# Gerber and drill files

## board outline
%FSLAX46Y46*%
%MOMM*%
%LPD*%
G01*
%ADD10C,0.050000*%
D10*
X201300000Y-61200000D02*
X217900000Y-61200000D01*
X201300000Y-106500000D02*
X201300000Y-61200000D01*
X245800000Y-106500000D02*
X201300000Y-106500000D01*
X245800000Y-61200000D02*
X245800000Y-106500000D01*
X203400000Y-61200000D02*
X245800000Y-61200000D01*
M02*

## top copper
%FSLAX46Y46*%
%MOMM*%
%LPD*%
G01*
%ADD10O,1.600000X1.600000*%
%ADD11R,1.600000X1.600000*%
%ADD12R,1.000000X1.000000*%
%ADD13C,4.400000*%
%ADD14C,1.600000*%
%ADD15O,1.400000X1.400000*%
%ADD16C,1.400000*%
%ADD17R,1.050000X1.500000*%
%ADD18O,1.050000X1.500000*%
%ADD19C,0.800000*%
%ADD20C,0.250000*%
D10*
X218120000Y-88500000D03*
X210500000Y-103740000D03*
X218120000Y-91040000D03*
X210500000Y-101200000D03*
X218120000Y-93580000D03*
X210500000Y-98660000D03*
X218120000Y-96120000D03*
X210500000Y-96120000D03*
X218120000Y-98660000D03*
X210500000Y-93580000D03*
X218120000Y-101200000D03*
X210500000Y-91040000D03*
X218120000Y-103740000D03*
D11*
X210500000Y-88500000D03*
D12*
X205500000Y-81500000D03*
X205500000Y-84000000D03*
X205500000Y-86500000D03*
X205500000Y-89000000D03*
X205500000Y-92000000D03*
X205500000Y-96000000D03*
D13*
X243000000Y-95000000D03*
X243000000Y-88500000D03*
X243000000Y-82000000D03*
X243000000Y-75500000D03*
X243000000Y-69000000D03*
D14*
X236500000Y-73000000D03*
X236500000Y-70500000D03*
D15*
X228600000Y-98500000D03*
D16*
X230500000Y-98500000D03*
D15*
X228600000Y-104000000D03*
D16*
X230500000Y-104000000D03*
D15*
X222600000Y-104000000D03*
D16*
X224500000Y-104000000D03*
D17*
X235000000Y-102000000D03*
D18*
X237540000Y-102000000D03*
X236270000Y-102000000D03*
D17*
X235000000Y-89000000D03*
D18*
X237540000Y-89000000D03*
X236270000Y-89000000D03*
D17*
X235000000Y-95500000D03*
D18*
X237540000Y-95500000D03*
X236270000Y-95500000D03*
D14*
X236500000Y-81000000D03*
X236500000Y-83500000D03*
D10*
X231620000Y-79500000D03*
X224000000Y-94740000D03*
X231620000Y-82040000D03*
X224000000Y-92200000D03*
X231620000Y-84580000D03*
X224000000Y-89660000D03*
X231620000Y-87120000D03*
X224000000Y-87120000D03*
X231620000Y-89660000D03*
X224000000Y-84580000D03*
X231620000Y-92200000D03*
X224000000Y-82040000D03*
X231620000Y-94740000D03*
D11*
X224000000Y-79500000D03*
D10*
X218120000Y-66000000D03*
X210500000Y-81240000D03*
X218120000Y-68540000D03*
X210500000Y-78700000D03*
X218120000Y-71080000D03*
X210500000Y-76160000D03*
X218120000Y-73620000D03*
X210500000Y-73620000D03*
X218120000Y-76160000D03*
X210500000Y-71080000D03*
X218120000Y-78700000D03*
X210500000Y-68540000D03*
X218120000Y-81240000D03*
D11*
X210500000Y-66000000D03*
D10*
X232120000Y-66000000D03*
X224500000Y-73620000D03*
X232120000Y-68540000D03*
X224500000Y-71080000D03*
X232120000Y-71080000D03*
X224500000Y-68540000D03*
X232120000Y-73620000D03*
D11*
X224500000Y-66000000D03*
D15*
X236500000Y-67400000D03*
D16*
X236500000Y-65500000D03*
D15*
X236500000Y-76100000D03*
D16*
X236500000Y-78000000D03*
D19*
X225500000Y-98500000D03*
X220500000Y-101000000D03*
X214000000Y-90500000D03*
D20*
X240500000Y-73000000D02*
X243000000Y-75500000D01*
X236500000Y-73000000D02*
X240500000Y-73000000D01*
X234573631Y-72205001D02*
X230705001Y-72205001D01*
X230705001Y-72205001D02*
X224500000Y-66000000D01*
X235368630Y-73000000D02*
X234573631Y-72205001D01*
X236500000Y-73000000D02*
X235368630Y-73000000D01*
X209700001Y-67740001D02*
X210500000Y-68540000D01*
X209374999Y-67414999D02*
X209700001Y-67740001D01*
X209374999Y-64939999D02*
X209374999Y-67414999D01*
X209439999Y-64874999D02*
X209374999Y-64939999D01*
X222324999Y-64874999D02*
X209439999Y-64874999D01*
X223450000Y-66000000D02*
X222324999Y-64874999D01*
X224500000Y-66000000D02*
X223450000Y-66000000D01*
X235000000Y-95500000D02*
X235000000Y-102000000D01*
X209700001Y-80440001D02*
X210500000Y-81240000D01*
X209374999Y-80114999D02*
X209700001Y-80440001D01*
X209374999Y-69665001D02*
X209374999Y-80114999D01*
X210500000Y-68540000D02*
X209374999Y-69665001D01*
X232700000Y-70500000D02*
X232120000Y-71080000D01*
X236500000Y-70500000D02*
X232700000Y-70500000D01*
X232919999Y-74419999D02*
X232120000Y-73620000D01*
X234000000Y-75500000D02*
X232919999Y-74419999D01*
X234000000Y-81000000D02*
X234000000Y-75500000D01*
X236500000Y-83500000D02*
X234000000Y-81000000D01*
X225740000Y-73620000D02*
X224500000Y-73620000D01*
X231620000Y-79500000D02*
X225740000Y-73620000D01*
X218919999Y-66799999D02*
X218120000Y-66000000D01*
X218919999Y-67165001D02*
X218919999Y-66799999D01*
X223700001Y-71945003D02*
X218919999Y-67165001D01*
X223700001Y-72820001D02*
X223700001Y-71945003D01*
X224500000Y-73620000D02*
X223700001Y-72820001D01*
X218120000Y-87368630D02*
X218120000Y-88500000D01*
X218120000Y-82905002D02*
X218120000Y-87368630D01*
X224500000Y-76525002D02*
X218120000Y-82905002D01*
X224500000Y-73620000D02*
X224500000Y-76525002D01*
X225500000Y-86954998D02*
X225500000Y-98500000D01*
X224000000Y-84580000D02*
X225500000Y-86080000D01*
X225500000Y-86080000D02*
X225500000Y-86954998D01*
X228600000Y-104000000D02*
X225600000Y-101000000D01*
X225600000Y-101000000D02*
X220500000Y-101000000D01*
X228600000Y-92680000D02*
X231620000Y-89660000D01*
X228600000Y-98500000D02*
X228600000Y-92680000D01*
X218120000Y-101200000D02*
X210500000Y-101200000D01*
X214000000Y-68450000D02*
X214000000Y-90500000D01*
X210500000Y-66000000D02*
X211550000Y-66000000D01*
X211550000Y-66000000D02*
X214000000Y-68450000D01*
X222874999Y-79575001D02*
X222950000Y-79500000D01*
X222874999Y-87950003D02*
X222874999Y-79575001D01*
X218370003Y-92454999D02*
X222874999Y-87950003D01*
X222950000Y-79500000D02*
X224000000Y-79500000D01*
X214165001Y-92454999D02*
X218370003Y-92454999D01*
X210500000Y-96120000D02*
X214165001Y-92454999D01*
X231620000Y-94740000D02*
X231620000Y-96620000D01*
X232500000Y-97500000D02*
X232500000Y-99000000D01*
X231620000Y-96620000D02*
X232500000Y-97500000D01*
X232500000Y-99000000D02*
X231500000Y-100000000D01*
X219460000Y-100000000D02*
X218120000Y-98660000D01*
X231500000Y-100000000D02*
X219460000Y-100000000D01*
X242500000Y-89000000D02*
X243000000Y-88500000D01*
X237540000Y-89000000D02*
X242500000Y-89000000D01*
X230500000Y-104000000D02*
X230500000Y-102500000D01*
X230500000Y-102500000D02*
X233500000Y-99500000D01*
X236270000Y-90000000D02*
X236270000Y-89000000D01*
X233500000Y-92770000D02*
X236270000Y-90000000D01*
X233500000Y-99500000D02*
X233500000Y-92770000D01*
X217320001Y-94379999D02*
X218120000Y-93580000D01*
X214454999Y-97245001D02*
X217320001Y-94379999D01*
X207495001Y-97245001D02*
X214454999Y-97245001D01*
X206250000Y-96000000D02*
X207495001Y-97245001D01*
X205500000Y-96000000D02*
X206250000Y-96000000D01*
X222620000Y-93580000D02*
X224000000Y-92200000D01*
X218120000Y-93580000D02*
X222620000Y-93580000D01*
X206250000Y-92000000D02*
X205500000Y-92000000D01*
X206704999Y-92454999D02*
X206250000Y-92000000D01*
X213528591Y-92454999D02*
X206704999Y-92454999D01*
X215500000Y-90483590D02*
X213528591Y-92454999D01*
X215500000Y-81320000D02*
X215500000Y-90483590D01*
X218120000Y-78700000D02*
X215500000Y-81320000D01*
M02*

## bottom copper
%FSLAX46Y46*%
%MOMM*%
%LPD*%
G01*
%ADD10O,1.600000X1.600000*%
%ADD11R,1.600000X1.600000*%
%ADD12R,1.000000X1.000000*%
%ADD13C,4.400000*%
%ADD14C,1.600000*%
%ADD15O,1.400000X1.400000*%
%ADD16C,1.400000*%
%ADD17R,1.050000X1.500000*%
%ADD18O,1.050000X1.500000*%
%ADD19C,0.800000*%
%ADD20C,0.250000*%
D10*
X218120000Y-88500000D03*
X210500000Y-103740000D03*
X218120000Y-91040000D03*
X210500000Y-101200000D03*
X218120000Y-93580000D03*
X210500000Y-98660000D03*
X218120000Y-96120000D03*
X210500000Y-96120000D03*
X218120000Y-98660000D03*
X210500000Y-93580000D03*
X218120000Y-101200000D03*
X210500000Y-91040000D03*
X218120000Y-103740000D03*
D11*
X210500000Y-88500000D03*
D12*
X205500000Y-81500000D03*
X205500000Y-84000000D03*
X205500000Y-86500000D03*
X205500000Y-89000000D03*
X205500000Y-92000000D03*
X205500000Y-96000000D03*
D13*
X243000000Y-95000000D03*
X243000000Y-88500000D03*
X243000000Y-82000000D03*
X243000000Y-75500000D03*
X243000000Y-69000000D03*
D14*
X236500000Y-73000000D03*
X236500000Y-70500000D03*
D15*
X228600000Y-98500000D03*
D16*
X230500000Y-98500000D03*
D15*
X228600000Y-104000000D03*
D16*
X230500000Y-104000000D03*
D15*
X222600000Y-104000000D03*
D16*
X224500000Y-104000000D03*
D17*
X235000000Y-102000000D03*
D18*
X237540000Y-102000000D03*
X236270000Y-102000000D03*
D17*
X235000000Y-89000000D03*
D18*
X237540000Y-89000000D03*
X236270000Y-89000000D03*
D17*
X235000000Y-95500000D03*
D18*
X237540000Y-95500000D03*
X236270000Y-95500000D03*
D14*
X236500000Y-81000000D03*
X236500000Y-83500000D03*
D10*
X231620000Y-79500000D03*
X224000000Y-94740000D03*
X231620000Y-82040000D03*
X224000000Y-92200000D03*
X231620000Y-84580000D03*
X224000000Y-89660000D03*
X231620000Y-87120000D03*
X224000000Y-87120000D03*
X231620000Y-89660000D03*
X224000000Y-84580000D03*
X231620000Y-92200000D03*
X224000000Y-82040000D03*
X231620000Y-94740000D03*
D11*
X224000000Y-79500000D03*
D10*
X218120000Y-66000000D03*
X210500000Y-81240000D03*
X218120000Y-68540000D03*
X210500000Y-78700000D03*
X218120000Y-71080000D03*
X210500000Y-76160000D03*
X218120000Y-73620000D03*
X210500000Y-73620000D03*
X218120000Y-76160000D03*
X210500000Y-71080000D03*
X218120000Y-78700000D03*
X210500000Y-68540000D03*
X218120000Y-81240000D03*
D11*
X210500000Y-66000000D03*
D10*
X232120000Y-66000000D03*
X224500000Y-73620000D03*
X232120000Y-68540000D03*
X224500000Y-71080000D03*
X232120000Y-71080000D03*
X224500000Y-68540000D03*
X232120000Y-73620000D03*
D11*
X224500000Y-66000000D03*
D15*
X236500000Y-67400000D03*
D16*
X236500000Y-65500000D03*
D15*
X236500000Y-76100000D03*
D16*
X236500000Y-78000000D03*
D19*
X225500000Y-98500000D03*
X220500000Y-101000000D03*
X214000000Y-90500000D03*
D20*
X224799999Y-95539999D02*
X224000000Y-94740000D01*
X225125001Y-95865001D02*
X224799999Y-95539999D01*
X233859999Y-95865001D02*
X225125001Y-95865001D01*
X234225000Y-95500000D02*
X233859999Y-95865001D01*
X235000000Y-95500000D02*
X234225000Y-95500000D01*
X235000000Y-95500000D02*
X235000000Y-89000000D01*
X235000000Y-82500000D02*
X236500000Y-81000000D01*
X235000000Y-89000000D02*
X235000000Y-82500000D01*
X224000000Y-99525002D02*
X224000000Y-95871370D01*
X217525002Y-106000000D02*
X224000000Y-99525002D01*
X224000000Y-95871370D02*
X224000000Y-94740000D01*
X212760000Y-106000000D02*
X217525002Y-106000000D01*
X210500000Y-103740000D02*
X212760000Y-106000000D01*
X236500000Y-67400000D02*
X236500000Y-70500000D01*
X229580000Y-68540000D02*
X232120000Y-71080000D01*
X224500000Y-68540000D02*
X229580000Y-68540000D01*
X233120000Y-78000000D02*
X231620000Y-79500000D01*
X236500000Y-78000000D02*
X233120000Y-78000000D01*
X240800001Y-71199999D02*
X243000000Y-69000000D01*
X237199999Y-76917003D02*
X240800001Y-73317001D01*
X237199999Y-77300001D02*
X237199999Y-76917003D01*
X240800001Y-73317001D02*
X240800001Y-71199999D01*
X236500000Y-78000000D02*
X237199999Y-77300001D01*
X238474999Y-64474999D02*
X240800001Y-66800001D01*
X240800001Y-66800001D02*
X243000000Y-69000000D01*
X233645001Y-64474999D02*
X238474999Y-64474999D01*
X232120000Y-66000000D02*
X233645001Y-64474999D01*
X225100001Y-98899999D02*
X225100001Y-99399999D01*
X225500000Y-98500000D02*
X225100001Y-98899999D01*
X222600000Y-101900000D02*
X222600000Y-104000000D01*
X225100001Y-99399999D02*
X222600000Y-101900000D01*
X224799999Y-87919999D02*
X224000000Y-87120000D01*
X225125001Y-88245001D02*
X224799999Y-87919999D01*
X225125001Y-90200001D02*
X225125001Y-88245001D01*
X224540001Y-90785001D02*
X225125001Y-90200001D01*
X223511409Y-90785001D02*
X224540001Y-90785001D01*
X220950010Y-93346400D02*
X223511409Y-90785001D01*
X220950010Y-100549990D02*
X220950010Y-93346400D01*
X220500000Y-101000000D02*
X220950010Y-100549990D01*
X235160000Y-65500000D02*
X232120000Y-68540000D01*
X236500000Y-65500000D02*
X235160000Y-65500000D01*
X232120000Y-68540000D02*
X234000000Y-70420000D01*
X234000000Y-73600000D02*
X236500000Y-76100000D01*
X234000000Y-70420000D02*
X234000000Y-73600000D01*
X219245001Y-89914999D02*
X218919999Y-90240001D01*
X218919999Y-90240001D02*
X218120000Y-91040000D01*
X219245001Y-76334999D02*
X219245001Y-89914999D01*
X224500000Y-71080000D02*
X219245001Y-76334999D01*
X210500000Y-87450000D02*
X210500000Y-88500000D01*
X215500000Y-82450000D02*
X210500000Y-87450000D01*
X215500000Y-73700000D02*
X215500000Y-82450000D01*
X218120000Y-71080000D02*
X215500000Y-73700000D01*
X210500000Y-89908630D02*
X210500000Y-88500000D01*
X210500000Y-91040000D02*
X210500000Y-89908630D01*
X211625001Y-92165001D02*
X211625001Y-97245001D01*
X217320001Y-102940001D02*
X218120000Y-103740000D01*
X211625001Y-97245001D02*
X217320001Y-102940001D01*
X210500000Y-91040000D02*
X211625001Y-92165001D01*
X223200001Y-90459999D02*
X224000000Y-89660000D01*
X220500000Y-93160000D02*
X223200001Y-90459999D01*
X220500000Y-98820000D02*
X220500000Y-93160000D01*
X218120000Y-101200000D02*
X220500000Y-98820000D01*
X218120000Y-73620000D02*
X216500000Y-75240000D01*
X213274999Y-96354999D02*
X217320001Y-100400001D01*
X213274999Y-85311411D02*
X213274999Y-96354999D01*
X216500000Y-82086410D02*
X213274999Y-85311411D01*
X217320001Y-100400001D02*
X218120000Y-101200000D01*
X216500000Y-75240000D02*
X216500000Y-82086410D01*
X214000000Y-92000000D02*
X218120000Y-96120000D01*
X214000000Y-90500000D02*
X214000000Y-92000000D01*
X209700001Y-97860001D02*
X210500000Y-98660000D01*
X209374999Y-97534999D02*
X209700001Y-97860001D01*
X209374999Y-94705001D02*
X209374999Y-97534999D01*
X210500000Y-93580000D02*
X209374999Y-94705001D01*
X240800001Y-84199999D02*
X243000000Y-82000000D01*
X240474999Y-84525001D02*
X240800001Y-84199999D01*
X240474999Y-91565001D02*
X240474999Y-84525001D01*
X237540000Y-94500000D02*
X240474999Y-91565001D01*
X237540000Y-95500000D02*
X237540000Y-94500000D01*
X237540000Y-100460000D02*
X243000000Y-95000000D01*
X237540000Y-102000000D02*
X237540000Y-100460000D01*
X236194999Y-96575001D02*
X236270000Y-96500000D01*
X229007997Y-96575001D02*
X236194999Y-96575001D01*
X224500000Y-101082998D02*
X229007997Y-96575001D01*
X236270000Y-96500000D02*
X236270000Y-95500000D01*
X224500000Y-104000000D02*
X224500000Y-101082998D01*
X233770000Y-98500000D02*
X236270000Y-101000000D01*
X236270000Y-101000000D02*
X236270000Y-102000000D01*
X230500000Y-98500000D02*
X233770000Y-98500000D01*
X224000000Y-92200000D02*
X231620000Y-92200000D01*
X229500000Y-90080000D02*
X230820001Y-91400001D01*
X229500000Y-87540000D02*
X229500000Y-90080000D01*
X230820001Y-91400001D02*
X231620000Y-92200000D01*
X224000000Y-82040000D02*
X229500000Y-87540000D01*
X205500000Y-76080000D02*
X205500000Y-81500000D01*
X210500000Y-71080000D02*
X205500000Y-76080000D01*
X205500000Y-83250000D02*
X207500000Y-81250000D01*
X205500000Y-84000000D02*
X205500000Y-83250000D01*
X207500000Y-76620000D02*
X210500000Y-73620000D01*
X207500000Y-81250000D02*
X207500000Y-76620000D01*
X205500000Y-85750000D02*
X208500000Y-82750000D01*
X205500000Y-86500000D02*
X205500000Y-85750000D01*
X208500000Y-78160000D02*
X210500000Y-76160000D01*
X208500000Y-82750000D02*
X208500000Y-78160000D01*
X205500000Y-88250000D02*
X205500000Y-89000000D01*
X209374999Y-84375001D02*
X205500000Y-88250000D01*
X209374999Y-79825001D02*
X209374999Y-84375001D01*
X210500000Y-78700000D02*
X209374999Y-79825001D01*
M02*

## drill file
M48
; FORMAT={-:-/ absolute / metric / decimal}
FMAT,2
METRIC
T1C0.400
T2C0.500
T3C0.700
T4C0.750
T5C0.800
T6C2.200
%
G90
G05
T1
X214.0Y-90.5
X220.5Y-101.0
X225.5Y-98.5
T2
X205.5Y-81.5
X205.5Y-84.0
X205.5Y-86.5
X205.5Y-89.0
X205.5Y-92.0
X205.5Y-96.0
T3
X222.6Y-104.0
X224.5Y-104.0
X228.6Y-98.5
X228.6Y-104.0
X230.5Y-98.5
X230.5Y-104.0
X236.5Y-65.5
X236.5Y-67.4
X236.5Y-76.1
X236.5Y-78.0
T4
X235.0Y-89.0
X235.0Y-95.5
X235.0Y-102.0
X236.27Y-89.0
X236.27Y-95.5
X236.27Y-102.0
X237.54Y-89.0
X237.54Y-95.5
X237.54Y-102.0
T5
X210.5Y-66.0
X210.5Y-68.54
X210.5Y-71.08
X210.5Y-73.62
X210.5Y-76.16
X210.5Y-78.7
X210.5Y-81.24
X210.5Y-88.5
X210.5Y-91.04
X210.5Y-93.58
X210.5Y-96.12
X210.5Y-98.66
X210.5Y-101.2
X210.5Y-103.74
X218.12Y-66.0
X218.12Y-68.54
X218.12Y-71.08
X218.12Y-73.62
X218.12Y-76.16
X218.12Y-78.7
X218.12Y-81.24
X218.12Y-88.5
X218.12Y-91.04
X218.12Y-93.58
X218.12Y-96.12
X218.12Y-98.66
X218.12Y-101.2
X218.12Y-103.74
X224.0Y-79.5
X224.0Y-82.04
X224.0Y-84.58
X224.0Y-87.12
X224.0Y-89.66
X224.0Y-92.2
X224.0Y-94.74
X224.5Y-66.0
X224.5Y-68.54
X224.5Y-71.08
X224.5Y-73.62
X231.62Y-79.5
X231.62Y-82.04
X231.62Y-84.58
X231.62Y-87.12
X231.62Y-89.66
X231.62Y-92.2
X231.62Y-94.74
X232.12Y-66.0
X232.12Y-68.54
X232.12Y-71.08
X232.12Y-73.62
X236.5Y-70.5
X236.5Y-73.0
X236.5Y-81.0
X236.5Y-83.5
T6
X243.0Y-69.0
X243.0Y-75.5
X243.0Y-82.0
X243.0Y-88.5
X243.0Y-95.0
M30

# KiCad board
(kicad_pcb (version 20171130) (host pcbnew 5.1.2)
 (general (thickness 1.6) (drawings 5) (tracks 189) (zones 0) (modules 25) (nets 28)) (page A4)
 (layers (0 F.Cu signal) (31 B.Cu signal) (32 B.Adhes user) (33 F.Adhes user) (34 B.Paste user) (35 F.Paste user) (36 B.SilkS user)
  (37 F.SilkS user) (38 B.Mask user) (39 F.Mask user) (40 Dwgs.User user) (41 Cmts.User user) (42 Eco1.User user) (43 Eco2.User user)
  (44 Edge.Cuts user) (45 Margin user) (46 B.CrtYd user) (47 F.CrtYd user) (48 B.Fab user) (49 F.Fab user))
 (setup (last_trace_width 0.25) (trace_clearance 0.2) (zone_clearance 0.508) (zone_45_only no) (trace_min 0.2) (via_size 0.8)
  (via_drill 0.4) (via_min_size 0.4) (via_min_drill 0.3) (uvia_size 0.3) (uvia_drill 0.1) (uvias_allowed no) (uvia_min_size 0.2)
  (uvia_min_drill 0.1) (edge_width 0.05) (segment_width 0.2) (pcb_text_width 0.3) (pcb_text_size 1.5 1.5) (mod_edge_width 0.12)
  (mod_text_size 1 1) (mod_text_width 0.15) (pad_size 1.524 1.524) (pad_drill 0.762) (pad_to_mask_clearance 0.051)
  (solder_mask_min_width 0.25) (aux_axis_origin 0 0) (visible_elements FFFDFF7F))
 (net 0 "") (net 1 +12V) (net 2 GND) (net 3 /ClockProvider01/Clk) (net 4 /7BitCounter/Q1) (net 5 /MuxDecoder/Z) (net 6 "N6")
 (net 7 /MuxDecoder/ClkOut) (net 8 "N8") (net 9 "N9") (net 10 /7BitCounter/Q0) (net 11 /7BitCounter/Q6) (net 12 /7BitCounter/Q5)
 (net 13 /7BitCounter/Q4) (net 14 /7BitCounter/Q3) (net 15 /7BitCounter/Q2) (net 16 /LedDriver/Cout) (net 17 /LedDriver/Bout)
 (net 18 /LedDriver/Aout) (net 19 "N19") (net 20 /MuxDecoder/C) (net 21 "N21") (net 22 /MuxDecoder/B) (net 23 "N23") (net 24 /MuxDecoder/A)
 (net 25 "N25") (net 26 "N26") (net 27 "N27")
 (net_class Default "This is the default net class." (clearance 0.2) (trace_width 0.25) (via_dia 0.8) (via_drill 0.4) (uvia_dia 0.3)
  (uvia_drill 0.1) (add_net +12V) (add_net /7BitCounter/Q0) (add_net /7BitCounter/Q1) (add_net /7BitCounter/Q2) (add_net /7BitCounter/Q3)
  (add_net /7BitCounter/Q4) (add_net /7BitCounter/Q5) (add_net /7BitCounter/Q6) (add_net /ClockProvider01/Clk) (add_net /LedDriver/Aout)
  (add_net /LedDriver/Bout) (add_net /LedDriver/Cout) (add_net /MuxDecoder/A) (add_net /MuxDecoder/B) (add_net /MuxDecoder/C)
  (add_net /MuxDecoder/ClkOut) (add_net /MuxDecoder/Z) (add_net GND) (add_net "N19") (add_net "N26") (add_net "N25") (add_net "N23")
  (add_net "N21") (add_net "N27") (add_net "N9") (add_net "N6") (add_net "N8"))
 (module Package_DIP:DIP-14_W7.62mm (layer F.Cu) (at 210.5 88.5)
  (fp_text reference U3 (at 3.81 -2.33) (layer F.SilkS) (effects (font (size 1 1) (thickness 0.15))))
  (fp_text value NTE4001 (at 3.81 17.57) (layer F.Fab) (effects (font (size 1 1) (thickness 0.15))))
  (pad 14 thru_hole oval (at 7.62 0) (size 1.6 1.6) (drill 0.8) (layers *.Cu *.Mask) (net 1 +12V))
  (pad 7 thru_hole oval (at 0 15.24) (size 1.6 1.6) (drill 0.8) (layers *.Cu *.Mask) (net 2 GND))
  (pad 13 thru_hole oval (at 7.62 2.54) (size 1.6 1.6) (drill 0.8) (layers *.Cu *.Mask) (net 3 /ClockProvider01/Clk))
  (pad 6 thru_hole oval (at 0 12.7) (size 1.6 1.6) (drill 0.8) (layers *.Cu *.Mask) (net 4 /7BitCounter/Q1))
  (pad 12 thru_hole oval (at 7.62 5.08) (size 1.6 1.6) (drill 0.8) (layers *.Cu *.Mask) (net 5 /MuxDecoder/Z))
  (pad 5 thru_hole oval (at 0 10.16) (size 1.6 1.6) (drill 0.8) (layers *.Cu *.Mask) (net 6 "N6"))
  (pad 11 thru_hole oval (at 7.62 7.62) (size 1.6 1.6) (drill 0.8) (layers *.Cu *.Mask) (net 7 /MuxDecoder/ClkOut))
  (pad 4 thru_hole oval (at 0 7.62) (size 1.6 1.6) (drill 0.8) (layers *.Cu *.Mask) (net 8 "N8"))
  (pad 10 thru_hole oval (at 7.62 10.16) (size 1.6 1.6) (drill 0.8) (layers *.Cu *.Mask) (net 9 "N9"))
  (pad 3 thru_hole oval (at 0 5.08) (size 1.6 1.6) (drill 0.8) (layers *.Cu *.Mask) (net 6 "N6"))
  (pad 9 thru_hole oval (at 7.62 12.7) (size 1.6 1.6) (drill 0.8) (layers *.Cu *.Mask) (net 4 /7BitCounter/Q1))
  (pad 2 thru_hole oval (at 0 2.54) (size 1.6 1.6) (drill 0.8) (layers *.Cu *.Mask) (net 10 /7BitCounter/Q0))
  (pad 8 thru_hole oval (at 7.62 15.24) (size 1.6 1.6) (drill 0.8) (layers *.Cu *.Mask) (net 10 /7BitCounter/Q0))
  (pad 1 thru_hole rect (at 0 0) (size 1.6 1.6) (drill 0.8) (layers *.Cu *.Mask) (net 10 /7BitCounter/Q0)))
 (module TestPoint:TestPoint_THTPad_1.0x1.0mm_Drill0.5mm (layer F.Cu) (at 205.5 81.5 180)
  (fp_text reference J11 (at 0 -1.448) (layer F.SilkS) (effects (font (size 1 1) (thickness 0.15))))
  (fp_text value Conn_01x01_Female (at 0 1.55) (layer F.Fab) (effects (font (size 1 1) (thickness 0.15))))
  (pad 1 thru_hole rect (at 0 0 180) (size 1 1) (drill 0.5) (layers *.Cu *.Mask) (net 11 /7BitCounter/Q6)))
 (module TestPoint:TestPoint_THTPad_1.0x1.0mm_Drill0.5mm (layer F.Cu) (at 205.5 84 180)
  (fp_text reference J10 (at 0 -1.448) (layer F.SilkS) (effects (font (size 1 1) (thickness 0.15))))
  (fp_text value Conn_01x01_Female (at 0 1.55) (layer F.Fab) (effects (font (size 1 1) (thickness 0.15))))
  (pad 1 thru_hole rect (at 0 0 180) (size 1 1) (drill 0.5) (layers *.Cu *.Mask) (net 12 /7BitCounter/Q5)))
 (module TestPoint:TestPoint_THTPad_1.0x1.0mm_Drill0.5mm (layer F.Cu) (at 205.5 86.5 180)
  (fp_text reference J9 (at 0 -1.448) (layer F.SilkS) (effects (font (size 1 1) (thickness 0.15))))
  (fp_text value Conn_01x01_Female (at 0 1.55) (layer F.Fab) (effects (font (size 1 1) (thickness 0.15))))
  (pad 1 thru_hole rect (at 0 0 180) (size 1 1) (drill 0.5) (layers *.Cu *.Mask) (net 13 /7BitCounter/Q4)))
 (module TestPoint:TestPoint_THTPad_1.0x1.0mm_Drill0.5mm (layer F.Cu) (at 205.5 89 180)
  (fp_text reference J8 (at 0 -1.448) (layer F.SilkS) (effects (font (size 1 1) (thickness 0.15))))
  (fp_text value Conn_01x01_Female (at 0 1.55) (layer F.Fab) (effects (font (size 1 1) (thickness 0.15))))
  (pad 1 thru_hole rect (at 0 0 180) (size 1 1) (drill 0.5) (layers *.Cu *.Mask) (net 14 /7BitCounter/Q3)))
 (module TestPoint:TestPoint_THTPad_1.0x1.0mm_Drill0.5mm (layer F.Cu) (at 205.5 92 180)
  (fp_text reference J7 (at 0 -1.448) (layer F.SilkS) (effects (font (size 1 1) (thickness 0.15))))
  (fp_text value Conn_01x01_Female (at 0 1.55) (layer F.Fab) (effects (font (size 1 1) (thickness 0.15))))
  (pad 1 thru_hole rect (at 0 0 180) (size 1 1) (drill 0.5) (layers *.Cu *.Mask) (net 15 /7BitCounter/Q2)))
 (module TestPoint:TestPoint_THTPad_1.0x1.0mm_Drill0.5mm (layer F.Cu) (at 205.5 96 180)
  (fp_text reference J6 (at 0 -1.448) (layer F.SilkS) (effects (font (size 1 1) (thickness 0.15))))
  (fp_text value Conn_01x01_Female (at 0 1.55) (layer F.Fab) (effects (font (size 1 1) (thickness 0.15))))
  (pad 1 thru_hole rect (at 0 0 180) (size 1 1) (drill 0.5) (layers *.Cu *.Mask) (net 5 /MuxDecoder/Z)))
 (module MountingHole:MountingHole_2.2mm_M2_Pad (layer F.Cu) (at 243 95)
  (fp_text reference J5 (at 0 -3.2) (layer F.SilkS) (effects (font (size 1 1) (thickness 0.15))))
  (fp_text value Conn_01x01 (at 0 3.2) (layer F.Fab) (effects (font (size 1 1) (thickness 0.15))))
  (pad 1 thru_hole circle (at 0 0) (size 4.4 4.4) (drill 2.2) (layers *.Cu *.Mask) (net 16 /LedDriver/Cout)))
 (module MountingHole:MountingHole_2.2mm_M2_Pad (layer F.Cu) (at 243 88.5)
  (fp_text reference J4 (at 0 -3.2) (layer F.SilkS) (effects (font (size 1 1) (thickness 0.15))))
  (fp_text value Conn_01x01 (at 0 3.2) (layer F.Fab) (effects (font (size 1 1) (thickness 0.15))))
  (pad 1 thru_hole circle (at 0 0) (size 4.4 4.4) (drill 2.2) (layers *.Cu *.Mask) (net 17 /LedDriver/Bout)))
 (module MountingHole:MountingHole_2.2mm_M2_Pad (layer F.Cu) (at 243 82)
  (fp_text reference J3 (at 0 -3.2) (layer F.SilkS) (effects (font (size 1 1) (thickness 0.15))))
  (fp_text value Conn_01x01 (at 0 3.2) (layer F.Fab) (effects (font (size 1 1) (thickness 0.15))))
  (pad 1 thru_hole circle (at 0 0) (size 4.4 4.4) (drill 2.2) (layers *.Cu *.Mask) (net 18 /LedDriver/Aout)))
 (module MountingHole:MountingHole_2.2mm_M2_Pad (layer F.Cu) (at 243 75.5)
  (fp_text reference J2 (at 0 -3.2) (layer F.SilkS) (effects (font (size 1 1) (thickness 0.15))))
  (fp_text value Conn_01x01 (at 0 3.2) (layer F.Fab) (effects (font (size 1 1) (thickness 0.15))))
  (pad 1 thru_hole circle (at 0 0) (size 4.4 4.4) (drill 2.2) (layers *.Cu *.Mask) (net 2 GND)))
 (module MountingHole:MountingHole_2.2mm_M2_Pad (layer F.Cu) (at 243 69)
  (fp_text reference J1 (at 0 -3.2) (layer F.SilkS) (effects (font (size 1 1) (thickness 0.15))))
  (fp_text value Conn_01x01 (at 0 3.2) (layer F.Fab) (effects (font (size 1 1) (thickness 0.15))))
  (pad 1 thru_hole circle (at 0 0) (size 4.4 4.4) (drill 2.2) (layers *.Cu *.Mask) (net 1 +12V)))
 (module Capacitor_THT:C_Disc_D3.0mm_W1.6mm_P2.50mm (layer F.Cu) (at 236.5 70.5 270)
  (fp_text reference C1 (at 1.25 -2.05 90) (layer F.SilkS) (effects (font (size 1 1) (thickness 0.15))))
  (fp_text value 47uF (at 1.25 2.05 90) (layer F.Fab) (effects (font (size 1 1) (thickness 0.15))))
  (pad 2 thru_hole circle (at 2.5 0 270) (size 1.6 1.6) (drill 0.8) (layers *.Cu *.Mask) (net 2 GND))
  (pad 1 thru_hole circle (at 0 0 270) (size 1.6 1.6) (drill 0.8) (layers *.Cu *.Mask) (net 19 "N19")))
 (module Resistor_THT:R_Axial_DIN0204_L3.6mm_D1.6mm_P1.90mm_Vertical (layer F.Cu) (at 230.5 98.5 180)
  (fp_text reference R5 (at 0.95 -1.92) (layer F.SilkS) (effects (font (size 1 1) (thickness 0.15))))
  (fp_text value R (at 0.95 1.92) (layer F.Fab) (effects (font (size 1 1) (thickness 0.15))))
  (pad 2 thru_hole oval (at 1.9 0 180) (size 1.4 1.4) (drill 0.7) (layers *.Cu *.Mask) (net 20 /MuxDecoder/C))
  (pad 1 thru_hole circle (at 0 0 180) (size 1.4 1.4) (drill 0.7) (layers *.Cu *.Mask) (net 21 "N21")))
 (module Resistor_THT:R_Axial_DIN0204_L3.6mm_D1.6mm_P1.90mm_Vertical (layer F.Cu) (at 230.5 104 180)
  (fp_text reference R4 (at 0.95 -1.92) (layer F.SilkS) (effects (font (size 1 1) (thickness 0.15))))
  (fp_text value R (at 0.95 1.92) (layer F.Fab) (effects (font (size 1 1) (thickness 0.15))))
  (pad 2 thru_hole oval (at 1.9 0 180) (size 1.4 1.4) (drill 0.7) (layers *.Cu *.Mask) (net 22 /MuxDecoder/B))
  (pad 1 thru_hole circle (at 0 0 180) (size 1.4 1.4) (drill 0.7) (layers *.Cu *.Mask) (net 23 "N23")))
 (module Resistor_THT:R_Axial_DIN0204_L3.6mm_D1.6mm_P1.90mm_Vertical (layer F.Cu) (at 224.5 104 180)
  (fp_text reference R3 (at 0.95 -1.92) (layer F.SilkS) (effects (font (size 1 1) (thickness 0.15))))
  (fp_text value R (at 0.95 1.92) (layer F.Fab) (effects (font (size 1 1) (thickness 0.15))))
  (pad 2 thru_hole oval (at 1.9 0 180) (size 1.4 1.4) (drill 0.7) (layers *.Cu *.Mask) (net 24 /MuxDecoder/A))
  (pad 1 thru_hole circle (at 0 0 180) (size 1.4 1.4) (drill 0.7) (layers *.Cu *.Mask) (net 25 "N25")))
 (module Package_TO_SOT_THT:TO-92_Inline (layer F.Cu) (at 235 102)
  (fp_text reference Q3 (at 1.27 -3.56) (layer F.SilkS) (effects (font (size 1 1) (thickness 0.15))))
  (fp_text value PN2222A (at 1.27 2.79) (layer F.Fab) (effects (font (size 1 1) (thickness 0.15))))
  (pad 1 thru_hole rect (at 0 0) (size 1.05 1.5) (drill 0.75) (layers *.Cu *.Mask) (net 2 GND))
  (pad 3 thru_hole oval (at 2.54 0) (size 1.05 1.5) (drill 0.75) (layers *.Cu *.Mask) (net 16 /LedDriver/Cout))
  (pad 2 thru_hole oval (at 1.27 0) (size 1.05 1.5) (drill 0.75) (layers *.Cu *.Mask) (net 21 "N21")))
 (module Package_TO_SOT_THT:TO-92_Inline (layer F.Cu) (at 235 89)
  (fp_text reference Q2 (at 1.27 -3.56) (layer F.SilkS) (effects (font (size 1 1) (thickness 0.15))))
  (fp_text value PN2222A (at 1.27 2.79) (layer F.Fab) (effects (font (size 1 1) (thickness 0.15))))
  (pad 1 thru_hole rect (at 0 0) (size 1.05 1.5) (drill 0.75) (layers *.Cu *.Mask) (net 2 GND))
  (pad 3 thru_hole oval (at 2.54 0) (size 1.05 1.5) (drill 0.75) (layers *.Cu *.Mask) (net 17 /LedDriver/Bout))
  (pad 2 thru_hole oval (at 1.27 0) (size 1.05 1.5) (drill 0.75) (layers *.Cu *.Mask) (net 23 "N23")))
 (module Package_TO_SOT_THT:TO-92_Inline (layer F.Cu) (at 235 95.5)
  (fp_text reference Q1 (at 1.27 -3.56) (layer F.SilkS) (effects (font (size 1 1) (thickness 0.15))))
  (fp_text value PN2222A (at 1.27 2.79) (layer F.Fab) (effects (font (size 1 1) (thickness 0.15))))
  (pad 1 thru_hole rect (at 0 0) (size 1.05 1.5) (drill 0.75) (layers *.Cu *.Mask) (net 2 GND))
  (pad 3 thru_hole oval (at 2.54 0) (size 1.05 1.5) (drill 0.75) (layers *.Cu *.Mask) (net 18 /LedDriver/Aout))
  (pad 2 thru_hole oval (at 1.27 0) (size 1.05 1.5) (drill 0.75) (layers *.Cu *.Mask) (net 25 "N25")))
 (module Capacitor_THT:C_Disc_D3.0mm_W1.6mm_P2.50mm (layer F.Cu) (at 236.5 83.5 90)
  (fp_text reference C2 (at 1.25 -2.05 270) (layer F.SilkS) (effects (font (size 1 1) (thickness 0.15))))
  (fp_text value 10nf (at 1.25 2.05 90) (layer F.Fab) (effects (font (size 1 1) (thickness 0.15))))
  (pad 2 thru_hole circle (at 2.5 0 90) (size 1.6 1.6) (drill 0.8) (layers *.Cu *.Mask) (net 2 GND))
  (pad 1 thru_hole circle (at 0 0 90) (size 1.6 1.6) (drill 0.8) (layers *.Cu *.Mask) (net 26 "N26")))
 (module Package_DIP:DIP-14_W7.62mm (layer F.Cu) (at 224 79.5)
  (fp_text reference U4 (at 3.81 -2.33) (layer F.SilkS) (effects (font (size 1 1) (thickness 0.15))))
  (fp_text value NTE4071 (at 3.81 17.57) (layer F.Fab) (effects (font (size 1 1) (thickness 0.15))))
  (pad 14 thru_hole oval (at 7.62 0) (size 1.6 1.6) (drill 0.8) (layers *.Cu *.Mask) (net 1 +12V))
  (pad 7 thru_hole oval (at 0 15.24) (size 1.6 1.6) (drill 0.8) (layers *.Cu *.Mask) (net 2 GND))
  (pad 13 thru_hole oval (at 7.62 2.54) (size 1.6 1.6) (drill 0.8) (layers *.Cu *.Mask))
  (pad 6 thru_hole oval (at 0 12.7) (size 1.6 1.6) (drill 0.8) (layers *.Cu *.Mask) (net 5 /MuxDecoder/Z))
  (pad 12 thru_hole oval (at 7.62 5.08) (size 1.6 1.6) (drill 0.8) (layers *.Cu *.Mask))
  (pad 5 thru_hole oval (at 0 10.16) (size 1.6 1.6) (drill 0.8) (layers *.Cu *.Mask) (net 4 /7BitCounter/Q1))
  (pad 11 thru_hole oval (at 7.62 7.62) (size 1.6 1.6) (drill 0.8) (layers *.Cu *.Mask))
  (pad 4 thru_hole oval (at 0 7.62) (size 1.6 1.6) (drill 0.8) (layers *.Cu *.Mask) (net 22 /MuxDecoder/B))
  (pad 10 thru_hole oval (at 7.62 10.16) (size 1.6 1.6) (drill 0.8) (layers *.Cu *.Mask) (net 20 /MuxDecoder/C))
  (pad 3 thru_hole oval (at 0 5.08) (size 1.6 1.6) (drill 0.8) (layers *.Cu *.Mask) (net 24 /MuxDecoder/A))
  (pad 9 thru_hole oval (at 7.62 12.7) (size 1.6 1.6) (drill 0.8) (layers *.Cu *.Mask) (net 5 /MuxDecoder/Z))
  (pad 2 thru_hole oval (at 0 2.54) (size 1.6 1.6) (drill 0.8) (layers *.Cu *.Mask) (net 5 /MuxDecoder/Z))
  (pad 8 thru_hole oval (at 7.62 15.24) (size 1.6 1.6) (drill 0.8) (layers *.Cu *.Mask) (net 9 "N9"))
  (pad 1 thru_hole rect (at 0 0) (size 1.6 1.6) (drill 0.8) (layers *.Cu *.Mask) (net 8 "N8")))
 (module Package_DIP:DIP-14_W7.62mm (layer F.Cu) (at 210.5 66)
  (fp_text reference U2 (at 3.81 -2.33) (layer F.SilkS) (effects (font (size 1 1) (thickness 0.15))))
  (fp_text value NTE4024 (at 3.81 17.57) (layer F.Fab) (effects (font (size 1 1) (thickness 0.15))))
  (pad 14 thru_hole oval (at 7.62 0) (size 1.6 1.6) (drill 0.8) (layers *.Cu *.Mask) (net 1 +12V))
  (pad 7 thru_hole oval (at 0 15.24) (size 1.6 1.6) (drill 0.8) (layers *.Cu *.Mask) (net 2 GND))
  (pad 13 thru_hole oval (at 7.62 2.54) (size 1.6 1.6) (drill 0.8) (layers *.Cu *.Mask))
  (pad 6 thru_hole oval (at 0 12.7) (size 1.6 1.6) (drill 0.8) (layers *.Cu *.Mask) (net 14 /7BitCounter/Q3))
  (pad 12 thru_hole oval (at 7.62 5.08) (size 1.6 1.6) (drill 0.8) (layers *.Cu *.Mask) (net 10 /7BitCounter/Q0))
  (pad 5 thru_hole oval (at 0 10.16) (size 1.6 1.6) (drill 0.8) (layers *.Cu *.Mask) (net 13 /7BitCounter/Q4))
  (pad 11 thru_hole oval (at 7.62 7.62) (size 1.6 1.6) (drill 0.8) (layers *.Cu *.Mask) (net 4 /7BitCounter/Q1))
  (pad 4 thru_hole oval (at 0 7.62) (size 1.6 1.6) (drill 0.8) (layers *.Cu *.Mask) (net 12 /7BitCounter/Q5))
  (pad 10 thru_hole oval (at 7.62 10.16) (size 1.6 1.6) (drill 0.8) (layers *.Cu *.Mask))
  (pad 3 thru_hole oval (at 0 5.08) (size 1.6 1.6) (drill 0.8) (layers *.Cu *.Mask) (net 11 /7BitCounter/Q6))
  (pad 9 thru_hole oval (at 7.62 12.7) (size 1.6 1.6) (drill 0.8) (layers *.Cu *.Mask) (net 15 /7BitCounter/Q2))
  (pad 2 thru_hole oval (at 0 2.54) (size 1.6 1.6) (drill 0.8) (layers *.Cu *.Mask) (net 2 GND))
  (pad 8 thru_hole oval (at 7.62 15.24) (size 1.6 1.6) (drill 0.8) (layers *.Cu *.Mask))
  (pad 1 thru_hole rect (at 0 0) (size 1.6 1.6) (drill 0.8) (layers *.Cu *.Mask) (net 7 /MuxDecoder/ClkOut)))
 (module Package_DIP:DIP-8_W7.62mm (layer F.Cu) (at 224.5 66)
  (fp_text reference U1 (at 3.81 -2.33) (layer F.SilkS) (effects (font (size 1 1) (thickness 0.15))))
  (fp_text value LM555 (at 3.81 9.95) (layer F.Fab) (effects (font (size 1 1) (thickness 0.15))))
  (pad 8 thru_hole oval (at 7.62 0) (size 1.6 1.6) (drill 0.8) (layers *.Cu *.Mask) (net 1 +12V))
  (pad 4 thru_hole oval (at 0 7.62) (size 1.6 1.6) (drill 0.8) (layers *.Cu *.Mask) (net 1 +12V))
  (pad 7 thru_hole oval (at 7.62 2.54) (size 1.6 1.6) (drill 0.8) (layers *.Cu *.Mask) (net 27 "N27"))
  (pad 3 thru_hole oval (at 0 5.08) (size 1.6 1.6) (drill 0.8) (layers *.Cu *.Mask) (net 3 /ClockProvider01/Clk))
  (pad 6 thru_hole oval (at 7.62 5.08) (size 1.6 1.6) (drill 0.8) (layers *.Cu *.Mask) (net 19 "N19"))
  (pad 2 thru_hole oval (at 0 2.54) (size 1.6 1.6) (drill 0.8) (layers *.Cu *.Mask) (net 19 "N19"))
  (pad 5 thru_hole oval (at 7.62 7.62) (size 1.6 1.6) (drill 0.8) (layers *.Cu *.Mask) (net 26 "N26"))
  (pad 1 thru_hole rect (at 0 0) (size 1.6 1.6) (drill 0.8) (layers *.Cu *.Mask) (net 2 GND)))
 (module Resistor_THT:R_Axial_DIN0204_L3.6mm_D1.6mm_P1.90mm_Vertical (layer F.Cu) (at 236.5 65.5 270)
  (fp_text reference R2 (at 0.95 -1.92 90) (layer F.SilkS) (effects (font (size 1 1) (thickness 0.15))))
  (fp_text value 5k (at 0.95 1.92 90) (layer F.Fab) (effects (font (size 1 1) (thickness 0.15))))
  (pad 2 thru_hole oval (at 1.9 0 270) (size 1.4 1.4) (drill 0.7) (layers *.Cu *.Mask) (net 19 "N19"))
  (pad 1 thru_hole circle (at 0 0 270) (size 1.4 1.4) (drill 0.7) (layers *.Cu *.Mask) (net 27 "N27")))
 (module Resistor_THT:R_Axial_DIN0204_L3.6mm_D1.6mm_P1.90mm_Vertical (layer F.Cu) (at 236.5 78 90)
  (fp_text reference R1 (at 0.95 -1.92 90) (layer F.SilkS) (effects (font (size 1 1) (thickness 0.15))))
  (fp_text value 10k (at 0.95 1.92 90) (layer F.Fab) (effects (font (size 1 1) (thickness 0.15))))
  (pad 2 thru_hole oval (at 1.9 0 90) (size 1.4 1.4) (drill 0.7) (layers *.Cu *.Mask) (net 27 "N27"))
  (pad 1 thru_hole circle (at 0 0 90) (size 1.4 1.4) (drill 0.7) (layers *.Cu *.Mask) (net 1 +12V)))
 (gr_line (start 201.3 61.2) (end 217.9 61.2) (layer Edge.Cuts) (width 0.05))
 (gr_line (start 201.3 106.5) (end 201.3 61.2) (layer Edge.Cuts) (width 0.05))
 (gr_line (start 245.8 106.5) (end 201.3 106.5) (layer Edge.Cuts) (width 0.05))
 (gr_line (start 245.8 61.2) (end 245.8 106.5) (layer Edge.Cuts) (width 0.05))
 (gr_line (start 203.4 61.2) (end 245.8 61.2) (layer Edge.Cuts) (width 0.05))
 (segment (start 224.799999 95.539999) (end 224 94.74) (width 0.25) (layer B.Cu) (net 2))
 (segment (start 225.125001 95.865001) (end 224.799999 95.539999) (width 0.25) (layer B.Cu) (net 2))
 (segment (start 233.859999 95.865001) (end 225.125001 95.865001) (width 0.25) (layer B.Cu) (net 2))
 (segment (start 234.225 95.5) (end 233.859999 95.865001) (width 0.25) (layer B.Cu) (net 2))
 (segment (start 235 95.5) (end 234.225 95.5) (width 0.25) (layer B.Cu) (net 2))
 (segment (start 235 95.5) (end 235 89) (width 0.25) (layer B.Cu) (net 2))
 (segment (start 235 82.5) (end 236.5 81) (width 0.25) (layer B.Cu) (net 2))
 (segment (start 235 89) (end 235 82.5) (width 0.25) (layer B.Cu) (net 2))
 (segment (start 240.5 73) (end 243 75.5) (width 0.25) (layer F.Cu) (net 2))
 (segment (start 236.5 73) (end 240.5 73) (width 0.25) (layer F.Cu) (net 2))
 (segment (start 234.573631 72.205001) (end 230.705001 72.205001) (width 0.25) (layer F.Cu) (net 2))
 (segment (start 230.705001 72.205001) (end 224.5 66) (width 0.25) (layer F.Cu) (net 2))
 (segment (start 235.36863 73) (end 234.573631 72.205001) (width 0.25) (layer F.Cu) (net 2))
 (segment (start 236.5 73) (end 235.36863 73) (width 0.25) (layer F.Cu) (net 2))
 (segment (start 209.700001 67.740001) (end 210.5 68.54) (width 0.25) (layer F.Cu) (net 2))
 (segment (start 209.374999 67.414999) (end 209.700001 67.740001) (width 0.25) (layer F.Cu) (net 2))
 (segment (start 209.374999 64.939999) (end 209.374999 67.414999) (width 0.25) (layer F.Cu) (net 2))
 (segment (start 209.439999 64.874999) (end 209.374999 64.939999) (width 0.25) (layer F.Cu) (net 2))
 (segment (start 222.324999 64.874999) (end 209.439999 64.874999) (width 0.25) (layer F.Cu) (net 2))
 (segment (start 223.45 66) (end 222.324999 64.874999) (width 0.25) (layer F.Cu) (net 2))
 (segment (start 224.5 66) (end 223.45 66) (width 0.25) (layer F.Cu) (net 2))
 (segment (start 235 95.5) (end 235 102) (width 0.25) (layer F.Cu) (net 2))
 (segment (start 224 99.525002) (end 224 95.87137) (width 0.25) (layer B.Cu) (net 2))
 (segment (start 217.525002 106) (end 224 99.525002) (width 0.25) (layer B.Cu) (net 2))
 (segment (start 224 95.87137) (end 224 94.74) (width 0.25) (layer B.Cu) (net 2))
 (segment (start 212.76 106) (end 217.525002 106) (width 0.25) (layer B.Cu) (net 2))
 (segment (start 210.5 103.74) (end 212.76 106) (width 0.25) (layer B.Cu) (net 2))
 (segment (start 209.700001 80.440001) (end 210.5 81.24) (width 0.25) (layer F.Cu) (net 2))
 (segment (start 209.374999 80.114999) (end 209.700001 80.440001) (width 0.25) (layer F.Cu) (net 2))
 (segment (start 209.374999 69.665001) (end 209.374999 80.114999) (width 0.25) (layer F.Cu) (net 2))
 (segment (start 210.5 68.54) (end 209.374999 69.665001) (width 0.25) (layer F.Cu) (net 2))
 (segment (start 236.5 67.4) (end 236.5 70.5) (width 0.25) (layer B.Cu) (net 19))
 (segment (start 232.7 70.5) (end 232.12 71.08) (width 0.25) (layer F.Cu) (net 19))
 (segment (start 236.5 70.5) (end 232.7 70.5) (width 0.25) (layer F.Cu) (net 19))
 (segment (start 229.58 68.54) (end 232.12 71.08) (width 0.25) (layer B.Cu) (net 19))
 (segment (start 224.5 68.54) (end 229.58 68.54) (width 0.25) (layer B.Cu) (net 19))
 (segment (start 232.919999 74.419999) (end 232.12 73.62) (width 0.25) (layer F.Cu) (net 26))
 (segment (start 234 75.5) (end 232.919999 74.419999) (width 0.25) (layer F.Cu) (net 26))
 (segment (start 234 81) (end 234 75.5) (width 0.25) (layer F.Cu) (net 26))
 (segment (start 236.5 83.5) (end 234 81) (width 0.25) (layer F.Cu) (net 26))
 (segment (start 233.12 78) (end 231.62 79.5) (width 0.25) (layer B.Cu) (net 1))
 (segment (start 236.5 78) (end 233.12 78) (width 0.25) (layer B.Cu) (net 1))
 (segment (start 240.800001 71.199999) (end 243 69) (width 0.25) (layer B.Cu) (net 1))
 (segment (start 237.199999 76.917003) (end 240.800001 73.317001) (width 0.25) (layer B.Cu) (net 1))
 (segment (start 237.199999 77.300001) (end 237.199999 76.917003) (width 0.25) (layer B.Cu) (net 1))
 (segment (start 240.800001 73.317001) (end 240.800001 71.199999) (width 0.25) (layer B.Cu) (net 1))
 (segment (start 236.5 78) (end 237.199999 77.300001) (width 0.25) (layer B.Cu) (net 1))
 (segment (start 238.474999 64.474999) (end 240.800001 66.800001) (width 0.25) (layer B.Cu) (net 1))
 (segment (start 240.800001 66.800001) (end 243 69) (width 0.25) (layer B.Cu) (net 1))
 (segment (start 233.645001 64.474999) (end 238.474999 64.474999) (width 0.25) (layer B.Cu) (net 1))
 (segment (start 232.12 66) (end 233.645001 64.474999) (width 0.25) (layer B.Cu) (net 1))
 (segment (start 225.74 73.62) (end 224.5 73.62) (width 0.25) (layer F.Cu) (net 1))
 (segment (start 231.62 79.5) (end 225.74 73.62) (width 0.25) (layer F.Cu) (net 1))
 (segment (start 218.919999 66.799999) (end 218.12 66) (width 0.25) (layer F.Cu) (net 1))
 (segment (start 218.919999 67.165001) (end 218.919999 66.799999) (width 0.25) (layer F.Cu) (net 1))
 (segment (start 223.700001 71.945003) (end 218.919999 67.165001) (width 0.25) (layer F.Cu) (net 1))
 (segment (start 223.700001 72.820001) (end 223.700001 71.945003) (width 0.25) (layer F.Cu) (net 1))
 (segment (start 224.5 73.62) (end 223.700001 72.820001) (width 0.25) (layer F.Cu) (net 1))
 (segment (start 218.12 87.36863) (end 218.12 88.5) (width 0.25) (layer F.Cu) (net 1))
 (segment (start 218.12 82.905002) (end 218.12 87.36863) (width 0.25) (layer F.Cu) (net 1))
 (segment (start 224.5 76.525002) (end 218.12 82.905002) (width 0.25) (layer F.Cu) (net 1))
 (segment (start 224.5 73.62) (end 224.5 76.525002) (width 0.25) (layer F.Cu) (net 1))
 (segment (start 225.5 86.954998) (end 225.5 98.5) (width 0.25) (layer F.Cu) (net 24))
 (via (at 225.5 98.5) (size 0.8) (drill 0.4) (layers F.Cu B.Cu) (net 24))
 (segment (start 224 84.58) (end 225.5 86.08) (width 0.25) (layer F.Cu) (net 24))
 (segment (start 225.5 86.08) (end 225.5 86.954998) (width 0.25) (layer F.Cu) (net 24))
 (segment (start 225.100001 98.899999) (end 225.100001 99.399999) (width 0.25) (layer B.Cu) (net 24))
 (segment (start 225.5 98.5) (end 225.100001 98.899999) (width 0.25) (layer B.Cu) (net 24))
 (segment (start 222.6 101.9) (end 222.6 104) (width 0.25) (layer B.Cu) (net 24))
 (segment (start 225.100001 99.399999) (end 222.6 101.9) (width 0.25) (layer B.Cu) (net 24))
 (via (at 220.5 101) (size 0.8) (drill 0.4) (layers F.Cu B.Cu) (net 22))
 (segment (start 228.6 104) (end 225.6 101) (width 0.25) (layer F.Cu) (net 22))
 (segment (start 225.6 101) (end 220.5 101) (width 0.25) (layer F.Cu) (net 22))
 (segment (start 224.799999 87.919999) (end 224 87.12) (width 0.25) (layer B.Cu) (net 22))
 (segment (start 225.125001 88.245001) (end 224.799999 87.919999) (width 0.25) (layer B.Cu) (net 22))
 (segment (start 225.125001 90.200001) (end 225.125001 88.245001) (width 0.25) (layer B.Cu) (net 22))
 (segment (start 224.540001 90.785001) (end 225.125001 90.200001) (width 0.25) (layer B.Cu) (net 22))
 (segment (start 223.511409 90.785001) (end 224.540001 90.785001) (width 0.25) (layer B.Cu) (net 22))
 (segment (start 220.95001 93.3464) (end 223.511409 90.785001) (width 0.25) (layer B.Cu) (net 22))
 (segment (start 220.95001 100.54999) (end 220.95001 93.3464) (width 0.25) (layer B.Cu) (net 22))
 (segment (start 220.5 101) (end 220.95001 100.54999) (width 0.25) (layer B.Cu) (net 22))
 (segment (start 228.6 92.68) (end 231.62 89.66) (width 0.25) (layer F.Cu) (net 20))
 (segment (start 228.6 98.5) (end 228.6 92.68) (width 0.25) (layer F.Cu) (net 20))
 (segment (start 235.16 65.5) (end 232.12 68.54) (width 0.25) (layer B.Cu) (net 27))
 (segment (start 236.5 65.5) (end 235.16 65.5) (width 0.25) (layer B.Cu) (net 27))
 (segment (start 232.12 68.54) (end 234 70.42) (width 0.25) (layer B.Cu) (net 27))
 (segment (start 234 73.6) (end 236.5 76.1) (width 0.25) (layer B.Cu) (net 27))
 (segment (start 234 70.42) (end 234 73.6) (width 0.25) (layer B.Cu) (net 27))
 (segment (start 219.245001 89.914999) (end 218.919999 90.240001) (width 0.25) (layer B.Cu) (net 3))
 (segment (start 218.919999 90.240001) (end 218.12 91.04) (width 0.25) (layer B.Cu) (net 3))
 (segment (start 219.245001 76.334999) (end 219.245001 89.914999) (width 0.25) (layer B.Cu) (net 3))
 (segment (start 224.5 71.08) (end 219.245001 76.334999) (width 0.25) (layer B.Cu) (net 3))
 (segment (start 210.5 87.45) (end 210.5 88.5) (width 0.25) (layer B.Cu) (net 10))
 (segment (start 215.5 82.45) (end 210.5 87.45) (width 0.25) (layer B.Cu) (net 10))
 (segment (start 215.5 73.7) (end 215.5 82.45) (width 0.25) (layer B.Cu) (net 10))
 (segment (start 218.12 71.08) (end 215.5 73.7) (width 0.25) (layer B.Cu) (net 10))
 (segment (start 210.5 89.90863) (end 210.5 88.5) (width 0.25) (layer B.Cu) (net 10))
 (segment (start 210.5 91.04) (end 210.5 89.90863) (width 0.25) (layer B.Cu) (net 10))
 (segment (start 211.625001 92.165001) (end 211.625001 97.245001) (width 0.25) (layer B.Cu) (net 10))
 (segment (start 217.320001 102.940001) (end 218.12 103.74) (width 0.25) (layer B.Cu) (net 10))
 (segment (start 211.625001 97.245001) (end 217.320001 102.940001) (width 0.25) (layer B.Cu) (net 10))
 (segment (start 210.5 91.04) (end 211.625001 92.165001) (width 0.25) (layer B.Cu) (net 10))
 (segment (start 223.200001 90.459999) (end 224 89.66) (width 0.25) (layer B.Cu) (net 4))
 (segment (start 220.5 93.16) (end 223.200001 90.459999) (width 0.25) (layer B.Cu) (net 4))
 (segment (start 220.5 98.82) (end 220.5 93.16) (width 0.25) (layer B.Cu) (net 4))
 (segment (start 218.12 101.2) (end 220.5 98.82) (width 0.25) (layer B.Cu) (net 4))
 (segment (start 218.12 101.2) (end 210.5 101.2) (width 0.25) (layer F.Cu) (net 4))
 (segment (start 218.12 73.62) (end 216.5 75.24) (width 0.25) (layer B.Cu) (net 4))
 (segment (start 213.274999 96.354999) (end 217.320001 100.400001) (width 0.25) (layer B.Cu) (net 4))
 (segment (start 213.274999 85.311411) (end 213.274999 96.354999) (width 0.25) (layer B.Cu) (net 4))
 (segment (start 216.5 82.08641) (end 213.274999 85.311411) (width 0.25) (layer B.Cu) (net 4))
 (segment (start 217.320001 100.400001) (end 218.12 101.2) (width 0.25) (layer B.Cu) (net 4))
 (segment (start 216.5 75.24) (end 216.5 82.08641) (width 0.25) (layer B.Cu) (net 4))
 (via (at 214 90.5) (size 0.8) (drill 0.4) (layers F.Cu B.Cu) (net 7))
 (segment (start 214 68.45) (end 214 90.5) (width 0.25) (layer F.Cu) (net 7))
 (segment (start 210.5 66) (end 211.55 66) (width 0.25) (layer F.Cu) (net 7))
 (segment (start 211.55 66) (end 214 68.45) (width 0.25) (layer F.Cu) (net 7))
 (segment (start 214 92) (end 218.12 96.12) (width 0.25) (layer B.Cu) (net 7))
 (segment (start 214 90.5) (end 214 92) (width 0.25) (layer B.Cu) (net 7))
 (segment (start 209.700001 97.860001) (end 210.5 98.66) (width 0.25) (layer B.Cu) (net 6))
 (segment (start 209.374999 97.534999) (end 209.700001 97.860001) (width 0.25) (layer B.Cu) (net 6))
 (segment (start 209.374999 94.705001) (end 209.374999 97.534999) (width 0.25) (layer B.Cu) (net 6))
 (segment (start 210.5 93.58) (end 209.374999 94.705001) (width 0.25) (layer B.Cu) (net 6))
 (segment (start 222.874999 79.575001) (end 222.95 79.5) (width 0.25) (layer F.Cu) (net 8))
 (segment (start 222.874999 87.950003) (end 222.874999 79.575001) (width 0.25) (layer F.Cu) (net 8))
 (segment (start 218.370003 92.454999) (end 222.874999 87.950003) (width 0.25) (layer F.Cu) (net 8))
 (segment (start 222.95 79.5) (end 224 79.5) (width 0.25) (layer F.Cu) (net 8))
 (segment (start 214.165001 92.454999) (end 218.370003 92.454999) (width 0.25) (layer F.Cu) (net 8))
 (segment (start 210.5 96.12) (end 214.165001 92.454999) (width 0.25) (layer F.Cu) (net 8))
 (segment (start 231.62 94.74) (end 231.62 96.62) (width 0.25) (layer F.Cu) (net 9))
 (segment (start 232.5 97.5) (end 232.5 99) (width 0.25) (layer F.Cu) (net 9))
 (segment (start 231.62 96.62) (end 232.5 97.5) (width 0.25) (layer F.Cu) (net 9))
 (segment (start 232.5 99) (end 231.5 100) (width 0.25) (layer F.Cu) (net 9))
 (segment (start 219.46 100) (end 218.12 98.66) (width 0.25) (layer F.Cu) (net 9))
 (segment (start 231.5 100) (end 219.46 100) (width 0.25) (layer F.Cu) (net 9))
 (segment (start 240.800001 84.199999) (end 243 82) (width 0.25) (layer B.Cu) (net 18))
 (segment (start 240.474999 84.525001) (end 240.800001 84.199999) (width 0.25) (layer B.Cu) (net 18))
 (segment (start 240.474999 91.565001) (end 240.474999 84.525001) (width 0.25) (layer B.Cu) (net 18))
 (segment (start 237.54 94.5) (end 240.474999 91.565001) (width 0.25) (layer B.Cu) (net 18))
 (segment (start 237.54 95.5) (end 237.54 94.5) (width 0.25) (layer B.Cu) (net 18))
 (segment (start 242.5 89) (end 243 88.5) (width 0.25) (layer F.Cu) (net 17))
 (segment (start 237.54 89) (end 242.5 89) (width 0.25) (layer F.Cu) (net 17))
 (segment (start 237.54 100.46) (end 243 95) (width 0.25) (layer B.Cu) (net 16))
 (segment (start 237.54 102) (end 237.54 100.46) (width 0.25) (layer B.Cu) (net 16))
 (segment (start 236.194999 96.575001) (end 236.27 96.5) (width 0.25) (layer B.Cu) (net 25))
 (segment (start 229.007997 96.575001) (end 236.194999 96.575001) (width 0.25) (layer B.Cu) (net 25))
 (segment (start 224.5 101.082998) (end 229.007997 96.575001) (width 0.25) (layer B.Cu) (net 25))
 (segment (start 236.27 96.5) (end 236.27 95.5) (width 0.25) (layer B.Cu) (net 25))
 (segment (start 224.5 104) (end 224.5 101.082998) (width 0.25) (layer B.Cu) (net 25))
 (segment (start 230.5 104) (end 230.5 102.5) (width 0.25) (layer F.Cu) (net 23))
 (segment (start 230.5 102.5) (end 233.5 99.5) (width 0.25) (layer F.Cu) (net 23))
 (segment (start 236.27 90) (end 236.27 89) (width 0.25) (layer F.Cu) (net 23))
 (segment (start 233.5 92.77) (end 236.27 90) (width 0.25) (layer F.Cu) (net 23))
 (segment (start 233.5 99.5) (end 233.5 92.77) (width 0.25) (layer F.Cu) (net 23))
 (segment (start 233.77 98.5) (end 236.27 101) (width 0.25) (layer B.Cu) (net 21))
 (segment (start 236.27 101) (end 236.27 102) (width 0.25) (layer B.Cu) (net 21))
 (segment (start 230.5 98.5) (end 233.77 98.5) (width 0.25) (layer B.Cu) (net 21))
 (segment (start 217.320001 94.379999) (end 218.12 93.58) (width 0.25) (layer F.Cu) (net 5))
 (segment (start 214.454999 97.245001) (end 217.320001 94.379999) (width 0.25) (layer F.Cu) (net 5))
 (segment (start 207.495001 97.245001) (end 214.454999 97.245001) (width 0.25) (layer F.Cu) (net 5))
 (segment (start 206.25 96) (end 207.495001 97.245001) (width 0.25) (layer F.Cu) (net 5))
 (segment (start 205.5 96) (end 206.25 96) (width 0.25) (layer F.Cu) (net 5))
 (segment (start 222.62 93.58) (end 224 92.2) (width 0.25) (layer F.Cu) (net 5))
 (segment (start 218.12 93.58) (end 222.62 93.58) (width 0.25) (layer F.Cu) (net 5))
 (segment (start 224 92.2) (end 231.62 92.2) (width 0.25) (layer B.Cu) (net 5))
 (segment (start 229.5 90.08) (end 230.820001 91.400001) (width 0.25) (layer B.Cu) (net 5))
 (segment (start 229.5 87.54) (end 229.5 90.08) (width 0.25) (layer B.Cu) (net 5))
 (segment (start 230.820001 91.400001) (end 231.62 92.2) (width 0.25) (layer B.Cu) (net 5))
 (segment (start 224 82.04) (end 229.5 87.54) (width 0.25) (layer B.Cu) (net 5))
 (segment (start 205.5 76.08) (end 205.5 81.5) (width 0.25) (layer B.Cu) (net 11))
 (segment (start 210.5 71.08) (end 205.5 76.08) (width 0.25) (layer B.Cu) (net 11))
 (segment (start 205.5 83.25) (end 207.5 81.25) (width 0.25) (layer B.Cu) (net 12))
 (segment (start 205.5 84) (end 205.5 83.25) (width 0.25) (layer B.Cu) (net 12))
 (segment (start 207.5 76.62) (end 210.5 73.62) (width 0.25) (layer B.Cu) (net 12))
 (segment (start 207.5 81.25) (end 207.5 76.62) (width 0.25) (layer B.Cu) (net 12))
 (segment (start 205.5 85.75) (end 208.5 82.75) (width 0.25) (layer B.Cu) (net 13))
 (segment (start 205.5 86.5) (end 205.5 85.75) (width 0.25) (layer B.Cu) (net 13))
 (segment (start 208.5 78.16) (end 210.5 76.16) (width 0.25) (layer B.Cu) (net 13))
 (segment (start 208.5 82.75) (end 208.5 78.16) (width 0.25) (layer B.Cu) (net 13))
 (segment (start 205.5 88.25) (end 205.5 89) (width 0.25) (layer B.Cu) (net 14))
 (segment (start 209.374999 84.375001) (end 205.5 88.25) (width 0.25) (layer B.Cu) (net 14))
 (segment (start 209.374999 79.825001) (end 209.374999 84.375001) (width 0.25) (layer B.Cu) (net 14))
 (segment (start 210.5 78.7) (end 209.374999 79.825001) (width 0.25) (layer B.Cu) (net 14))
 (segment (start 206.25 92) (end 205.5 92) (width 0.25) (layer F.Cu) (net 15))
 (segment (start 206.704999 92.454999) (end 206.25 92) (width 0.25) (layer F.Cu) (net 15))
 (segment (start 213.528591 92.454999) (end 206.704999 92.454999) (width 0.25) (layer F.Cu) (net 15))
 (segment (start 215.5 90.48359) (end 213.528591 92.454999) (width 0.25) (layer F.Cu) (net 15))
 (segment (start 215.5 81.32) (end 215.5 90.48359) (width 0.25) (layer F.Cu) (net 15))
 (segment (start 218.12 78.7) (end 215.5 81.32) (width 0.25) (layer F.Cu) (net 15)))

